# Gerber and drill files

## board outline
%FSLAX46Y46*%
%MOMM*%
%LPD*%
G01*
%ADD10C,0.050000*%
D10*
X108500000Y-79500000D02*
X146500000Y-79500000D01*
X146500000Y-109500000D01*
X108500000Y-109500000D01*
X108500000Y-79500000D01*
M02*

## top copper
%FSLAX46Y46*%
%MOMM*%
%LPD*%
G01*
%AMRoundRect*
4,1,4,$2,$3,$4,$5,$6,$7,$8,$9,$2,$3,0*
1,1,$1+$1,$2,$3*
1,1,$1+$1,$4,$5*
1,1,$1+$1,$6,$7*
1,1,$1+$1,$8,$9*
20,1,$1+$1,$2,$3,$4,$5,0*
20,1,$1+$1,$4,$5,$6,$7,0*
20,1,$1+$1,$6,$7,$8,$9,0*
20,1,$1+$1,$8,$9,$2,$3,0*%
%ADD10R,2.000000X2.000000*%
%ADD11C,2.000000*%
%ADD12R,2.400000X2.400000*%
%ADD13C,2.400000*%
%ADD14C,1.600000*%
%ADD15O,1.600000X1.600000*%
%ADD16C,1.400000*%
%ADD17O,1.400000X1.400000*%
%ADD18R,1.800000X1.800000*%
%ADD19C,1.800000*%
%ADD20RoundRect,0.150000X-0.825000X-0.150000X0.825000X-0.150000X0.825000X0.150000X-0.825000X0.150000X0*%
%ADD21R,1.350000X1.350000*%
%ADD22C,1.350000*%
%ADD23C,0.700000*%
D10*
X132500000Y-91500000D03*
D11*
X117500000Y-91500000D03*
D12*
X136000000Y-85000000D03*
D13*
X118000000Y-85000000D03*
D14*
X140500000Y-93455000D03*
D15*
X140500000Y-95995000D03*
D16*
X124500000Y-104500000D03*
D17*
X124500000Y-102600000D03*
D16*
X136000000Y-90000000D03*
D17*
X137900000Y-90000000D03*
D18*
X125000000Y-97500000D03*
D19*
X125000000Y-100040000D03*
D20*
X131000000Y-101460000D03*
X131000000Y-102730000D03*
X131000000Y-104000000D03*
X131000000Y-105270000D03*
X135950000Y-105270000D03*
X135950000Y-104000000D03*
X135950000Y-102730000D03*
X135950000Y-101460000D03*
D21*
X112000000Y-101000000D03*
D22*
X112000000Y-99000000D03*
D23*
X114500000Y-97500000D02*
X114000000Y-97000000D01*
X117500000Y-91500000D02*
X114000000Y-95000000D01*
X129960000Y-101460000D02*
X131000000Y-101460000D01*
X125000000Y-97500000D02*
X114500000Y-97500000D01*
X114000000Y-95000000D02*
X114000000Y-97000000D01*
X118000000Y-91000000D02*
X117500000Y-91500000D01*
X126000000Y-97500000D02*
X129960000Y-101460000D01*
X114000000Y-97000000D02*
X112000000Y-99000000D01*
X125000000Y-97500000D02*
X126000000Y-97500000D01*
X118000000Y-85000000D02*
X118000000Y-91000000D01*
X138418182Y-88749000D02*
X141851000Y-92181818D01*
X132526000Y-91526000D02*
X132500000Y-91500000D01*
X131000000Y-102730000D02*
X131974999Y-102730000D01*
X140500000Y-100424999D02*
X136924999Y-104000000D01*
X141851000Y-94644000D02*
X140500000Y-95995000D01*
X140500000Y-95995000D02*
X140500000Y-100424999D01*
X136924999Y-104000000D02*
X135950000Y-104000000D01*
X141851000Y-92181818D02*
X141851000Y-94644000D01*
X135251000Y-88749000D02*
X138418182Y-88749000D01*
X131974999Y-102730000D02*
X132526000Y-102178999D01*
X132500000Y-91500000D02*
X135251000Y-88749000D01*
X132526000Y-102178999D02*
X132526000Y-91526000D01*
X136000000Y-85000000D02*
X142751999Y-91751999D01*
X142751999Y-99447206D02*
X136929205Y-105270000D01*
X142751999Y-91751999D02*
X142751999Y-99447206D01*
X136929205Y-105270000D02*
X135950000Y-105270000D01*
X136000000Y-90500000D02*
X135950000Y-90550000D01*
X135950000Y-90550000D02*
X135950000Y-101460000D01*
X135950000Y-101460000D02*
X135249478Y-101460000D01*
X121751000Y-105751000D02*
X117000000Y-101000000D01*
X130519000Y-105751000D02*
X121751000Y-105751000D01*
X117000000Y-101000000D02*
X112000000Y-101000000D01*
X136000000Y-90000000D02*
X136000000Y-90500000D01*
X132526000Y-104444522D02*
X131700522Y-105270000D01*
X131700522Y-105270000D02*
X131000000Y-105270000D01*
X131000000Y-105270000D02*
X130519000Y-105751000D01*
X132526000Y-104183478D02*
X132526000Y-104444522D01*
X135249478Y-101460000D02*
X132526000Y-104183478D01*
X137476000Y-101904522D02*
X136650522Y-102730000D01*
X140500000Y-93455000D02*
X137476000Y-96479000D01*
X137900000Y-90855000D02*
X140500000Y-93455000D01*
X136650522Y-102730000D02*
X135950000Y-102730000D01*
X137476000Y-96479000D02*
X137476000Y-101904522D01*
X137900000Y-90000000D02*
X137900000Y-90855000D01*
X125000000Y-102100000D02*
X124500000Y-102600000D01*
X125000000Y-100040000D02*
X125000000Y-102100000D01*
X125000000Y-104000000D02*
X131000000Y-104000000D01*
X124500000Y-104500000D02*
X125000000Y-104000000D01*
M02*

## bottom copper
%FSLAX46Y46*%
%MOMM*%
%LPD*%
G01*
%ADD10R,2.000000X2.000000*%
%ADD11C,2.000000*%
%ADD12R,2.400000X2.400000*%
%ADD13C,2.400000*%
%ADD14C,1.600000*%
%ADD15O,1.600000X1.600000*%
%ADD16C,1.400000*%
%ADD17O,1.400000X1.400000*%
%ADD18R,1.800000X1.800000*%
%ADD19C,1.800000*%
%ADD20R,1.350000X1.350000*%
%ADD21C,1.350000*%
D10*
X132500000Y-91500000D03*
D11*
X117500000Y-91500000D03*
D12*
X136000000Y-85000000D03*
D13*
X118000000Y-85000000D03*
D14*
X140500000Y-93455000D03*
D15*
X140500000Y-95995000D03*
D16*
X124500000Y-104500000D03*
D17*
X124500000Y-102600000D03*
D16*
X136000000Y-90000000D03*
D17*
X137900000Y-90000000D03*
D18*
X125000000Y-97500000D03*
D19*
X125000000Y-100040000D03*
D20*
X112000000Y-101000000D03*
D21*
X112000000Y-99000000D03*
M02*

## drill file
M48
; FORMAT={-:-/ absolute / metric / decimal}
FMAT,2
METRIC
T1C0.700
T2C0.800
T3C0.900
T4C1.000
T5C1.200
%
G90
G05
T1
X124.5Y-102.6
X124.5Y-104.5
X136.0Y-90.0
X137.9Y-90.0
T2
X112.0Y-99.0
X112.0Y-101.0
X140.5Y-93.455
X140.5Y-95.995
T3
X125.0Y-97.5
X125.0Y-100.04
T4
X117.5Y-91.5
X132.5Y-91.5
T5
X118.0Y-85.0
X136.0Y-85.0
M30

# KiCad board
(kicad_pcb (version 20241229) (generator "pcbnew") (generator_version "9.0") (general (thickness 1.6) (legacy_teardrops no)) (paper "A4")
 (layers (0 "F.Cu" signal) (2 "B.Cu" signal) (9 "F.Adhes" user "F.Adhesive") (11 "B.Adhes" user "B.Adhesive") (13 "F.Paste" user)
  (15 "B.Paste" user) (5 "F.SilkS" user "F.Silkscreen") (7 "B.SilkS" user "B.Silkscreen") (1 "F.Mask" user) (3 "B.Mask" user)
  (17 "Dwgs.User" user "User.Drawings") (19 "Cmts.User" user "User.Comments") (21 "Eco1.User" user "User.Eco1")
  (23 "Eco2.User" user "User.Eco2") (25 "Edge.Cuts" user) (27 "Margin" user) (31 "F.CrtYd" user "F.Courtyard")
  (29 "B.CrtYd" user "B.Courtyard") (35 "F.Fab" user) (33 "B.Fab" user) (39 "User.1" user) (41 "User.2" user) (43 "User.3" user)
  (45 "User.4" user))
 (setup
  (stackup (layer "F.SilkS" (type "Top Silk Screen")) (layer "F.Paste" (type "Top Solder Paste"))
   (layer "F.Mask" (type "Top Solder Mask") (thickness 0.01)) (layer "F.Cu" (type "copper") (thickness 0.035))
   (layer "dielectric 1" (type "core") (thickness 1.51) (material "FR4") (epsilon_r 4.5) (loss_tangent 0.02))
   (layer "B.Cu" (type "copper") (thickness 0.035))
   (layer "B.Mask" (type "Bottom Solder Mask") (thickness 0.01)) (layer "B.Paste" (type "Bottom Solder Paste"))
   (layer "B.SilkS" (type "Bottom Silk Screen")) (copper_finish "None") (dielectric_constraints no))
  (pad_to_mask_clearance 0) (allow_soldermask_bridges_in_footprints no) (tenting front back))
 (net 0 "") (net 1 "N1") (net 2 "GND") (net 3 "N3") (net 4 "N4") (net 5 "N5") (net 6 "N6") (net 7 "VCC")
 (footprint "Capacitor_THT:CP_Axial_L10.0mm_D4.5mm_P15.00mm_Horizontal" (layer "F.Cu") (at 132.5 91.5 180)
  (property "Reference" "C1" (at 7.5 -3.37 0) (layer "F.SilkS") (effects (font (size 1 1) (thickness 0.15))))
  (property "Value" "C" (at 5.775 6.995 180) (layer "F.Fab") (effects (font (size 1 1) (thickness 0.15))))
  (pad "1" thru_hole rect (at 0 0 180) (size 2 2) (drill 1) (layers "*.Cu" "*.Mask") (remove_unused_layers no) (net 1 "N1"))
  (pad "2" thru_hole circle (at 15 0 180) (size 2 2) (drill 1) (layers "*.Cu" "*.Mask") (remove_unused_layers no) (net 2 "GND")))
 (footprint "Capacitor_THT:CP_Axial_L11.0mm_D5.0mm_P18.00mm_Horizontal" (layer "F.Cu") (at 136 85 180)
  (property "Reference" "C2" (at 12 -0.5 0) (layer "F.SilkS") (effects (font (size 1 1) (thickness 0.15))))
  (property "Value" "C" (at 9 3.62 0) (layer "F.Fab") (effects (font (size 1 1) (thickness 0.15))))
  (pad "1" thru_hole rect (at 0 0 180) (size 2.4 2.4) (drill 1.2) (layers "*.Cu" "*.Mask") (remove_unused_layers no) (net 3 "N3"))
  (pad "2" thru_hole circle (at 18 0 180) (size 2.4 2.4) (drill 1.2) (layers "*.Cu" "*.Mask") (remove_unused_layers no) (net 2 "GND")))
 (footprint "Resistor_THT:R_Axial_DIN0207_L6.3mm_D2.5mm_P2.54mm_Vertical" (layer "F.Cu") (at 140.5 93.455 -90)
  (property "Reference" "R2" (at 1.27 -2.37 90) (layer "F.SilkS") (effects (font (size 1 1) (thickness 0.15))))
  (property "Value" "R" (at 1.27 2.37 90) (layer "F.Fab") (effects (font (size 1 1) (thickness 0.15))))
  (pad "1" thru_hole circle (at 0 0 270) (size 1.6 1.6) (drill 0.8) (layers "*.Cu" "*.Mask") (remove_unused_layers no) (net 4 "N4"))
  (pad "2" thru_hole oval (at 2.54 0 270) (size 1.6 1.6) (drill 0.8) (layers "*.Cu" "*.Mask") (remove_unused_layers no) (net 1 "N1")))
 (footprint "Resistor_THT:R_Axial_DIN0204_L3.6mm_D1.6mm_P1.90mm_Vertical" (layer "F.Cu") (at 124.5 104.5 90)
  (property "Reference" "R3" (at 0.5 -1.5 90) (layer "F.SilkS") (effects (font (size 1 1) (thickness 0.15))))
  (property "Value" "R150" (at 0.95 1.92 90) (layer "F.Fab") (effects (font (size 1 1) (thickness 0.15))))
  (pad "1" thru_hole circle (at 0 0 90) (size 1.4 1.4) (drill 0.7) (layers "*.Cu" "*.Mask") (remove_unused_layers no) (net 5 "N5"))
  (pad "2" thru_hole oval (at 1.9 0 90) (size 1.4 1.4) (drill 0.7) (layers "*.Cu" "*.Mask") (remove_unused_layers no) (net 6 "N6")))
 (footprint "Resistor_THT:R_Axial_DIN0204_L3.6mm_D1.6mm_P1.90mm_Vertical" (layer "F.Cu") (at 136 90)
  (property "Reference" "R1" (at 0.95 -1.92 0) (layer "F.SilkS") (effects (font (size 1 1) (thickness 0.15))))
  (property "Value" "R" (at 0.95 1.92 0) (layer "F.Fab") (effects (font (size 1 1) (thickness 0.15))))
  (pad "1" thru_hole circle (at 0 0) (size 1.4 1.4) (drill 0.7) (layers "*.Cu" "*.Mask") (remove_unused_layers no) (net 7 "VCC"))
  (pad "2" thru_hole oval (at 1.9 0) (size 1.4 1.4) (drill 0.7) (layers "*.Cu" "*.Mask") (remove_unused_layers no) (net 4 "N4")))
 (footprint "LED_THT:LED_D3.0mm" (layer "F.Cu") (at 125 97.5 -90)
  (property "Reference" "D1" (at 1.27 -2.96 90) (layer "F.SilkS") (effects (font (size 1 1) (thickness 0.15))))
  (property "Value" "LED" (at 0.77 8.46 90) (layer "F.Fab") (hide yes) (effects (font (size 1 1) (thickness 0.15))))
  (pad "1" thru_hole rect (at 0 0 270) (size 1.8 1.8) (drill 0.9) (layers "*.Cu" "*.Mask") (remove_unused_layers no) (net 2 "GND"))
  (pad "2" thru_hole circle (at 2.54 0 270) (size 1.8 1.8) (drill 0.9) (layers "*.Cu" "*.Mask") (remove_unused_layers no) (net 6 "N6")))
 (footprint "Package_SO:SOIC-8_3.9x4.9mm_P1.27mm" (layer "F.Cu") (at 133.475 103.365)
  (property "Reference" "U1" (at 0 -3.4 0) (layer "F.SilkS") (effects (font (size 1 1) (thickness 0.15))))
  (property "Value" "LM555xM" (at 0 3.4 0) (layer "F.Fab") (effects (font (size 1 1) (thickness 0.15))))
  (pad "1" smd roundrect (at -2.475 -1.905) (size 1.95 0.6) (layers "F.Cu" "F.Mask" "F.Paste") (roundrect_rratio 0.25) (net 2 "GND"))
  (pad "2" smd roundrect (at -2.475 -0.635) (size 1.95 0.6) (layers "F.Cu" "F.Mask" "F.Paste") (roundrect_rratio 0.25) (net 1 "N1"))
  (pad "3" smd roundrect (at -2.475 0.635) (size 1.95 0.6) (layers "F.Cu" "F.Mask" "F.Paste") (roundrect_rratio 0.25) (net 5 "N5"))
  (pad "4" smd roundrect (at -2.475 1.905) (size 1.95 0.6) (layers "F.Cu" "F.Mask" "F.Paste") (roundrect_rratio 0.25) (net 7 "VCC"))
  (pad "5" smd roundrect (at 2.475 1.905) (size 1.95 0.6) (layers "F.Cu" "F.Mask" "F.Paste") (roundrect_rratio 0.25) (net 3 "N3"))
  (pad "6" smd roundrect (at 2.475 0.635) (size 1.95 0.6) (layers "F.Cu" "F.Mask" "F.Paste") (roundrect_rratio 0.25) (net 1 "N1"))
  (pad "7" smd roundrect (at 2.475 -0.635) (size 1.95 0.6) (layers "F.Cu" "F.Mask" "F.Paste") (roundrect_rratio 0.25) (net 4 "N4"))
  (pad "8" smd roundrect (at 2.475 -1.905) (size 1.95 0.6) (layers "F.Cu" "F.Mask" "F.Paste") (roundrect_rratio 0.25) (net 7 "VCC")))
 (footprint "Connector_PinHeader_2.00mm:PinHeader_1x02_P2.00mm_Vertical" (layer "F.Cu") (at 112 101 180)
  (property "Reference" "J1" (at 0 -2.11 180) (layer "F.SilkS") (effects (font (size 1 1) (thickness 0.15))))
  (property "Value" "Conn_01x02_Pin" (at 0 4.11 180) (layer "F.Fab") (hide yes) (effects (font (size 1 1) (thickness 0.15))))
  (pad "1" thru_hole rect (at 0 0 180) (size 1.35 1.35) (drill 0.8) (layers "*.Cu" "*.Mask") (remove_unused_layers no) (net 7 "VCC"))
  (pad "2" thru_hole circle (at 0 2 180) (size 1.35 1.35) (drill 0.8) (layers "*.Cu" "*.Mask") (remove_unused_layers no) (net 2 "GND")))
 (gr_rect (start 108.5 79.5) (end 146.5 109.5) (stroke (width 0.05) (type default)) (fill no) (layer "Edge.Cuts"))
 (segment (start 114.5 97.5) (end 114 97) (width 0.7) (layer "F.Cu") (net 2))
 (segment (start 117.5 91.5) (end 114 95) (width 0.7) (layer "F.Cu") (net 2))
 (segment (start 129.96 101.46) (end 131 101.46) (width 0.7) (layer "F.Cu") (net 2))
 (segment (start 125 97.5) (end 114.5 97.5) (width 0.7) (layer "F.Cu") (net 2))
 (segment (start 114 95) (end 114 97) (width 0.7) (layer "F.Cu") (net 2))
 (segment (start 118 91) (end 117.5 91.5) (width 0.7) (layer "F.Cu") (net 2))
 (segment (start 126 97.5) (end 129.96 101.46) (width 0.7) (layer "F.Cu") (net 2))
 (segment (start 114 97) (end 112 99) (width 0.7) (layer "F.Cu") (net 2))
 (segment (start 125 97.5) (end 126 97.5) (width 0.7) (layer "F.Cu") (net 2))
 (segment (start 118 85) (end 118 91) (width 0.7) (layer "F.Cu") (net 2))
 (segment (start 138.418182 88.749) (end 141.851 92.181818) (width 0.7) (layer "F.Cu") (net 1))
 (segment (start 132.526 91.526) (end 132.5 91.5) (width 0.7) (layer "F.Cu") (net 1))
 (segment (start 131 102.73) (end 131.974999 102.73) (width 0.7) (layer "F.Cu") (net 1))
 (segment (start 140.5 100.424999) (end 136.924999 104) (width 0.7) (layer "F.Cu") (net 1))
 (segment (start 141.851 94.644) (end 140.5 95.995) (width 0.7) (layer "F.Cu") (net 1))
 (segment (start 140.5 95.995) (end 140.5 100.424999) (width 0.7) (layer "F.Cu") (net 1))
 (segment (start 136.924999 104) (end 135.95 104) (width 0.7) (layer "F.Cu") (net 1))
 (segment (start 141.851 92.181818) (end 141.851 94.644) (width 0.7) (layer "F.Cu") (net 1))
 (segment (start 135.251 88.749) (end 138.418182 88.749) (width 0.7) (layer "F.Cu") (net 1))
 (segment (start 131.974999 102.73) (end 132.526 102.178999) (width 0.7) (layer "F.Cu") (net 1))
 (segment (start 132.5 91.5) (end 135.251 88.749) (width 0.7) (layer "F.Cu") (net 1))
 (segment (start 132.526 102.178999) (end 132.526 91.526) (width 0.7) (layer "F.Cu") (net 1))
 (segment (start 136 85) (end 142.751999 91.751999) (width 0.7) (layer "F.Cu") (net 3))
 (segment (start 142.751999 99.447206) (end 136.929205 105.27) (width 0.7) (layer "F.Cu") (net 3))
 (segment (start 142.751999 91.751999) (end 142.751999 99.447206) (width 0.7) (layer "F.Cu") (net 3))
 (segment (start 136.929205 105.27) (end 135.95 105.27) (width 0.7) (layer "F.Cu") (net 3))
 (segment (start 136 90.5) (end 135.95 90.55) (width 0.7) (layer "F.Cu") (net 7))
 (segment (start 135.95 90.55) (end 135.95 101.46) (width 0.7) (layer "F.Cu") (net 7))
 (segment (start 135.95 101.46) (end 135.249478 101.46) (width 0.7) (layer "F.Cu") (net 7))
 (segment (start 121.751 105.751) (end 117 101) (width 0.7) (layer "F.Cu") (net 7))
 (segment (start 130.519 105.751) (end 121.751 105.751) (width 0.7) (layer "F.Cu") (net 7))
 (segment (start 117 101) (end 112 101) (width 0.7) (layer "F.Cu") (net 7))
 (segment (start 136 90) (end 136 90.5) (width 0.7) (layer "F.Cu") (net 7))
 (segment (start 132.526 104.444522) (end 131.700522 105.27) (width 0.7) (layer "F.Cu") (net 7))
 (segment (start 131.700522 105.27) (end 131 105.27) (width 0.7) (layer "F.Cu") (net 7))
 (segment (start 131 105.27) (end 130.519 105.751) (width 0.7) (layer "F.Cu") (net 7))
 (segment (start 132.526 104.183478) (end 132.526 104.444522) (width 0.7) (layer "F.Cu") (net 7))
 (segment (start 135.249478 101.46) (end 132.526 104.183478) (width 0.7) (layer "F.Cu") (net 7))
 (segment (start 137.476 101.904522) (end 136.650522 102.73) (width 0.7) (layer "F.Cu") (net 4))
 (segment (start 140.5 93.455) (end 137.476 96.479) (width 0.7) (layer "F.Cu") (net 4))
 (segment (start 137.9 90.855) (end 140.5 93.455) (width 0.7) (layer "F.Cu") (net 4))
 (segment (start 136.650522 102.73) (end 135.95 102.73) (width 0.7) (layer "F.Cu") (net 4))
 (segment (start 137.476 96.479) (end 137.476 101.904522) (width 0.7) (layer "F.Cu") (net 4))
 (segment (start 137.9 90) (end 137.9 90.855) (width 0.7) (layer "F.Cu") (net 4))
 (segment (start 125 102.1) (end 124.5 102.6) (width 0.7) (layer "F.Cu") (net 6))
 (segment (start 125 100.04) (end 125 102.1) (width 0.7) (layer "F.Cu") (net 6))
 (segment (start 125 104) (end 131 104) (width 0.7) (layer "F.Cu") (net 5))
 (segment (start 124.5 104.5) (end 125 104) (width 0.7) (layer "F.Cu") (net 5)))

